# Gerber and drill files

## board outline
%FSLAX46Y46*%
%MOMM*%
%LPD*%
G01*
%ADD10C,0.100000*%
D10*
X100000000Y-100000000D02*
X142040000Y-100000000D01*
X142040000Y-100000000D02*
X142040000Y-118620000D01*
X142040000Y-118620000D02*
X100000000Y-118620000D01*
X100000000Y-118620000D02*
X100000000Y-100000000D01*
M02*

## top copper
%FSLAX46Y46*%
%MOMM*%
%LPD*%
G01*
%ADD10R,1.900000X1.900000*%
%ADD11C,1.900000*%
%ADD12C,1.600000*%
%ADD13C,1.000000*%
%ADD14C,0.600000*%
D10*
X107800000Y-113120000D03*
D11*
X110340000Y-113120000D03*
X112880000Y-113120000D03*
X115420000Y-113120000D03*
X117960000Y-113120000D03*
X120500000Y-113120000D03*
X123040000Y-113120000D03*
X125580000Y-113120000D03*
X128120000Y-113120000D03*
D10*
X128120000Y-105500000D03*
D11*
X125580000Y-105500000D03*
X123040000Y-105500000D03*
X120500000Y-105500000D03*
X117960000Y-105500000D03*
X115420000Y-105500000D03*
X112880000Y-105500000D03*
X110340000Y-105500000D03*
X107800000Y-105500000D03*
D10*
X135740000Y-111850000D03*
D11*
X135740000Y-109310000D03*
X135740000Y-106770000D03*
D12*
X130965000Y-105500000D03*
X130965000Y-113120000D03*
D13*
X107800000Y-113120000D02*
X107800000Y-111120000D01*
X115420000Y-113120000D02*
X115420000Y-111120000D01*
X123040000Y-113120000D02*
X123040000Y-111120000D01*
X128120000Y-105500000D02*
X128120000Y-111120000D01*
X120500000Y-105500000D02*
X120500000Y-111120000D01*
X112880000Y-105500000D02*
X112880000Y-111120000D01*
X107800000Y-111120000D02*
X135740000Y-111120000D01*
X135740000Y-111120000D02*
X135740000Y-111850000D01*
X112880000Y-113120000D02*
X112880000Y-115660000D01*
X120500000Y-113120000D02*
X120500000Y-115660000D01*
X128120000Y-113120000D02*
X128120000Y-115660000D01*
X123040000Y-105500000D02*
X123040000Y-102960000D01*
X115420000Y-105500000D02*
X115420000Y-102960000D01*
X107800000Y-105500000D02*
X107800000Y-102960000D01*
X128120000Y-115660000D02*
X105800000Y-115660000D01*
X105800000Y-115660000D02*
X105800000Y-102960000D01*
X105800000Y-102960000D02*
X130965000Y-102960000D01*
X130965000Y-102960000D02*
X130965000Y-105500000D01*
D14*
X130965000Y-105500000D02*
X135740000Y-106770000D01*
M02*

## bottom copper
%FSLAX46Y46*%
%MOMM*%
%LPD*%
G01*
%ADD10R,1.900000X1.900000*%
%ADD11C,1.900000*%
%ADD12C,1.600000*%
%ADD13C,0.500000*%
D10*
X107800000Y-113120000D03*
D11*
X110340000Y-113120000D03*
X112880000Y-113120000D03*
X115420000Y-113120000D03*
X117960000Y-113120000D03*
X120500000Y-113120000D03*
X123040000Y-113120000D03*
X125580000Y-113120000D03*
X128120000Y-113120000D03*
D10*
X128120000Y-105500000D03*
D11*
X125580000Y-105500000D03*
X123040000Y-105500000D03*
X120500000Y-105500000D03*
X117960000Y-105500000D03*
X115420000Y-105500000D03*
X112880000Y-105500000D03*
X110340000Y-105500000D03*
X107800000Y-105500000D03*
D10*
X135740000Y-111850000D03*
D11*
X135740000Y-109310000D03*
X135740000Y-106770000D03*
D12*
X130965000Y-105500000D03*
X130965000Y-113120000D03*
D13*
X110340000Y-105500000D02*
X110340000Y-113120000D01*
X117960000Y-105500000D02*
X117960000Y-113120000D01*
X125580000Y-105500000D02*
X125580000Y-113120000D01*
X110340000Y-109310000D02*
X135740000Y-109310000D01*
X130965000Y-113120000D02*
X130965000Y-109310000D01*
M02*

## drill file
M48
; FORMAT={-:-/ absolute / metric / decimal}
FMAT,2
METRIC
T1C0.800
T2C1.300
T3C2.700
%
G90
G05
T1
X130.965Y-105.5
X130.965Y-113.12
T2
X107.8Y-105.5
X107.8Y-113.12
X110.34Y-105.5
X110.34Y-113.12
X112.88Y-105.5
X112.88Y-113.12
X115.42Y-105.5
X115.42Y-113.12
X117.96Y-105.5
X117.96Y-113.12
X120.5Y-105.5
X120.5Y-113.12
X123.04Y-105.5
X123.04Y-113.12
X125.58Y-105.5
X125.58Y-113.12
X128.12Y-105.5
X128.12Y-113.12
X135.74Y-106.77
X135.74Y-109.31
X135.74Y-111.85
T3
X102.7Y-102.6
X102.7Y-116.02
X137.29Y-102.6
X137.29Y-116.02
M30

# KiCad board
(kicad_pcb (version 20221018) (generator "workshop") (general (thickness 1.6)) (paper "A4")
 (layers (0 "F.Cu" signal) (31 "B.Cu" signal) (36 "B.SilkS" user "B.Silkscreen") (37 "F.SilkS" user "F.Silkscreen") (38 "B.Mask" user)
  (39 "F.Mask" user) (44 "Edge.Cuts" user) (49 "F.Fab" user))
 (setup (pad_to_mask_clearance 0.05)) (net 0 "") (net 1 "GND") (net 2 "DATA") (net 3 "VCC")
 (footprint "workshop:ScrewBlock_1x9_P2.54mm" (layer "F.Cu") (at 107.800 113.120 0)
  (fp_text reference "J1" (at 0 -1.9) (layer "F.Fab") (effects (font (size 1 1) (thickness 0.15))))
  (pad "1" thru_hole rect (at 0.000 0 0) (size 1.9 1.9) (drill 1.3) (layers "*.Cu" "*.Mask") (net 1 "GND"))
  (pad "2" thru_hole circle (at 2.540 0 0) (size 1.9 1.9) (drill 1.3) (layers "*.Cu" "*.Mask") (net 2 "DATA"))
  (pad "3" thru_hole circle (at 5.080 0 0) (size 1.9 1.9) (drill 1.3) (layers "*.Cu" "*.Mask") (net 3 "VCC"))
  (pad "4" thru_hole circle (at 7.620 0 0) (size 1.9 1.9) (drill 1.3) (layers "*.Cu" "*.Mask") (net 1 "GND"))
  (pad "5" thru_hole circle (at 10.160 0 0) (size 1.9 1.9) (drill 1.3) (layers "*.Cu" "*.Mask") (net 2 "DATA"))
  (pad "6" thru_hole circle (at 12.700 0 0) (size 1.9 1.9) (drill 1.3) (layers "*.Cu" "*.Mask") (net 3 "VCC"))
  (pad "7" thru_hole circle (at 15.240 0 0) (size 1.9 1.9) (drill 1.3) (layers "*.Cu" "*.Mask") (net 1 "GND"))
  (pad "8" thru_hole circle (at 17.780 0 0) (size 1.9 1.9) (drill 1.3) (layers "*.Cu" "*.Mask") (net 2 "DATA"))
  (pad "9" thru_hole circle (at 20.320 0 0) (size 1.9 1.9) (drill 1.3) (layers "*.Cu" "*.Mask") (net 3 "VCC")))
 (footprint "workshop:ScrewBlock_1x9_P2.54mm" (layer "F.Cu") (at 128.120 105.500 180)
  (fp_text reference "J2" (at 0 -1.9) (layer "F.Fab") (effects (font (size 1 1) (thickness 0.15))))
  (pad "1" thru_hole rect (at 0.000 0 180) (size 1.9 1.9) (drill 1.3) (layers "*.Cu" "*.Mask") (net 1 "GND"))
  (pad "2" thru_hole circle (at 2.540 0 180) (size 1.9 1.9) (drill 1.3) (layers "*.Cu" "*.Mask") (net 2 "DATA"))
  (pad "3" thru_hole circle (at 5.080 0 180) (size 1.9 1.9) (drill 1.3) (layers "*.Cu" "*.Mask") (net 3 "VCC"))
  (pad "4" thru_hole circle (at 7.620 0 180) (size 1.9 1.9) (drill 1.3) (layers "*.Cu" "*.Mask") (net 1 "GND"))
  (pad "5" thru_hole circle (at 10.160 0 180) (size 1.9 1.9) (drill 1.3) (layers "*.Cu" "*.Mask") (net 2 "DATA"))
  (pad "6" thru_hole circle (at 12.700 0 180) (size 1.9 1.9) (drill 1.3) (layers "*.Cu" "*.Mask") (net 3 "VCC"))
  (pad "7" thru_hole circle (at 15.240 0 180) (size 1.9 1.9) (drill 1.3) (layers "*.Cu" "*.Mask") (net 1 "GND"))
  (pad "8" thru_hole circle (at 17.780 0 180) (size 1.9 1.9) (drill 1.3) (layers "*.Cu" "*.Mask") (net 2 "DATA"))
  (pad "9" thru_hole circle (at 20.320 0 180) (size 1.9 1.9) (drill 1.3) (layers "*.Cu" "*.Mask") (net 3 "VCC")))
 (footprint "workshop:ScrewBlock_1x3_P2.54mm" (layer "F.Cu") (at 135.740 111.850 90)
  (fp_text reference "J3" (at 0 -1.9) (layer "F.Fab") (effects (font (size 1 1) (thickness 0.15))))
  (pad "1" thru_hole rect (at 0.000 0 90) (size 1.9 1.9) (drill 1.3) (layers "*.Cu" "*.Mask") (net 1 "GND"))
  (pad "2" thru_hole circle (at 2.540 0 90) (size 1.9 1.9) (drill 1.3) (layers "*.Cu" "*.Mask") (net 2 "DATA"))
  (pad "3" thru_hole circle (at 5.080 0 90) (size 1.9 1.9) (drill 1.3) (layers "*.Cu" "*.Mask") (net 3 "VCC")))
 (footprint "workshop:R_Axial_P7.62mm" (layer "F.Cu") (at 130.965 105.500)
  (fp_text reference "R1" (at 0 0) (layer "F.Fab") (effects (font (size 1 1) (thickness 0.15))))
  (pad "1" thru_hole circle (at 0.000 0.000) (size 1.6 1.6) (drill 0.8) (layers "*.Cu" "*.Mask") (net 3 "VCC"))
  (pad "2" thru_hole circle (at 0.000 7.620) (size 1.6 1.6) (drill 0.8) (layers "*.Cu" "*.Mask") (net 2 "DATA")))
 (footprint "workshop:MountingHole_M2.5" (layer "F.Cu") (at 102.700 102.600)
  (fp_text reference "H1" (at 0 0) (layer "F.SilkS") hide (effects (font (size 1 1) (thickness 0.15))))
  (pad "" np_thru_hole circle (at 0 0) (size 2.7 2.7) (drill 2.7) (layers "*.Cu" "*.Mask")))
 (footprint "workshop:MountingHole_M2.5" (layer "F.Cu") (at 102.700 116.020)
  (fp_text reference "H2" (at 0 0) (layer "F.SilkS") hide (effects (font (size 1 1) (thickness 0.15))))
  (pad "" np_thru_hole circle (at 0 0) (size 2.7 2.7) (drill 2.7) (layers "*.Cu" "*.Mask")))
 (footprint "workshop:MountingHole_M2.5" (layer "F.Cu") (at 137.290 102.600)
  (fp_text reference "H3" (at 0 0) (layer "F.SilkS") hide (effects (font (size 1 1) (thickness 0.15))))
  (pad "" np_thru_hole circle (at 0 0) (size 2.7 2.7) (drill 2.7) (layers "*.Cu" "*.Mask")))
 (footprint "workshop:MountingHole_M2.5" (layer "F.Cu") (at 137.290 116.020)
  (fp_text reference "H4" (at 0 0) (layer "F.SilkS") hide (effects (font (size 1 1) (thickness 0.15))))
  (pad "" np_thru_hole circle (at 0 0) (size 2.7 2.7) (drill 2.7) (layers "*.Cu" "*.Mask")))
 (segment (start 107.800 113.120) (end 107.800 111.120) (width 1.0) (layer "F.Cu") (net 1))
 (segment (start 115.420 113.120) (end 115.420 111.120) (width 1.0) (layer "F.Cu") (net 1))
 (segment (start 123.040 113.120) (end 123.040 111.120) (width 1.0) (layer "F.Cu") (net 1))
 (segment (start 128.120 105.500) (end 128.120 111.120) (width 1.0) (layer "F.Cu") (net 1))
 (segment (start 120.500 105.500) (end 120.500 111.120) (width 1.0) (layer "F.Cu") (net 1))
 (segment (start 112.880 105.500) (end 112.880 111.120) (width 1.0) (layer "F.Cu") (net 1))
 (segment (start 107.800 111.120) (end 135.740 111.120) (width 1.0) (layer "F.Cu") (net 1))
 (segment (start 135.740 111.120) (end 135.740 111.850) (width 1.0) (layer "F.Cu") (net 1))
 (segment (start 110.340 105.500) (end 110.340 113.120) (width 0.5) (layer "B.Cu") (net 2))
 (segment (start 117.960 105.500) (end 117.960 113.120) (width 0.5) (layer "B.Cu") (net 2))
 (segment (start 125.580 105.500) (end 125.580 113.120) (width 0.5) (layer "B.Cu") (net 2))
 (segment (start 110.340 109.310) (end 135.740 109.310) (width 0.5) (layer "B.Cu") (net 2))
 (segment (start 112.880 113.120) (end 112.880 115.660) (width 1.0) (layer "F.Cu") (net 3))
 (segment (start 120.500 113.120) (end 120.500 115.660) (width 1.0) (layer "F.Cu") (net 3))
 (segment (start 128.120 113.120) (end 128.120 115.660) (width 1.0) (layer "F.Cu") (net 3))
 (segment (start 123.040 105.500) (end 123.040 102.960) (width 1.0) (layer "F.Cu") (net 3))
 (segment (start 115.420 105.500) (end 115.420 102.960) (width 1.0) (layer "F.Cu") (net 3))
 (segment (start 107.800 105.500) (end 107.800 102.960) (width 1.0) (layer "F.Cu") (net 3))
 (segment (start 128.120 115.660) (end 105.800 115.660) (width 1.0) (layer "F.Cu") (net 3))
 (segment (start 105.800 115.660) (end 105.800 102.960) (width 1.0) (layer "F.Cu") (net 3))
 (segment (start 105.800 102.960) (end 130.965 102.960) (width 1.0) (layer "F.Cu") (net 3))
 (segment (start 130.965 102.960) (end 130.965 105.500) (width 1.0) (layer "F.Cu") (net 3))
 (segment (start 130.965 105.500) (end 135.740 106.770) (width 0.6) (layer "F.Cu") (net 3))
 (segment (start 130.965 113.120) (end 130.965 109.310) (width 0.5) (layer "B.Cu") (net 2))
 (gr_line (start 100.000 100.000) (end 142.040 100.000) (layer "Edge.Cuts") (width 0.1))
 (gr_line (start 142.040 100.000) (end 142.040 118.620) (layer "Edge.Cuts") (width 0.1))
 (gr_line (start 142.040 118.620) (end 100.000 118.620) (layer "Edge.Cuts") (width 0.1))
 (gr_line (start 100.000 118.620) (end 100.000 100.000) (layer "Edge.Cuts") (width 0.1)))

